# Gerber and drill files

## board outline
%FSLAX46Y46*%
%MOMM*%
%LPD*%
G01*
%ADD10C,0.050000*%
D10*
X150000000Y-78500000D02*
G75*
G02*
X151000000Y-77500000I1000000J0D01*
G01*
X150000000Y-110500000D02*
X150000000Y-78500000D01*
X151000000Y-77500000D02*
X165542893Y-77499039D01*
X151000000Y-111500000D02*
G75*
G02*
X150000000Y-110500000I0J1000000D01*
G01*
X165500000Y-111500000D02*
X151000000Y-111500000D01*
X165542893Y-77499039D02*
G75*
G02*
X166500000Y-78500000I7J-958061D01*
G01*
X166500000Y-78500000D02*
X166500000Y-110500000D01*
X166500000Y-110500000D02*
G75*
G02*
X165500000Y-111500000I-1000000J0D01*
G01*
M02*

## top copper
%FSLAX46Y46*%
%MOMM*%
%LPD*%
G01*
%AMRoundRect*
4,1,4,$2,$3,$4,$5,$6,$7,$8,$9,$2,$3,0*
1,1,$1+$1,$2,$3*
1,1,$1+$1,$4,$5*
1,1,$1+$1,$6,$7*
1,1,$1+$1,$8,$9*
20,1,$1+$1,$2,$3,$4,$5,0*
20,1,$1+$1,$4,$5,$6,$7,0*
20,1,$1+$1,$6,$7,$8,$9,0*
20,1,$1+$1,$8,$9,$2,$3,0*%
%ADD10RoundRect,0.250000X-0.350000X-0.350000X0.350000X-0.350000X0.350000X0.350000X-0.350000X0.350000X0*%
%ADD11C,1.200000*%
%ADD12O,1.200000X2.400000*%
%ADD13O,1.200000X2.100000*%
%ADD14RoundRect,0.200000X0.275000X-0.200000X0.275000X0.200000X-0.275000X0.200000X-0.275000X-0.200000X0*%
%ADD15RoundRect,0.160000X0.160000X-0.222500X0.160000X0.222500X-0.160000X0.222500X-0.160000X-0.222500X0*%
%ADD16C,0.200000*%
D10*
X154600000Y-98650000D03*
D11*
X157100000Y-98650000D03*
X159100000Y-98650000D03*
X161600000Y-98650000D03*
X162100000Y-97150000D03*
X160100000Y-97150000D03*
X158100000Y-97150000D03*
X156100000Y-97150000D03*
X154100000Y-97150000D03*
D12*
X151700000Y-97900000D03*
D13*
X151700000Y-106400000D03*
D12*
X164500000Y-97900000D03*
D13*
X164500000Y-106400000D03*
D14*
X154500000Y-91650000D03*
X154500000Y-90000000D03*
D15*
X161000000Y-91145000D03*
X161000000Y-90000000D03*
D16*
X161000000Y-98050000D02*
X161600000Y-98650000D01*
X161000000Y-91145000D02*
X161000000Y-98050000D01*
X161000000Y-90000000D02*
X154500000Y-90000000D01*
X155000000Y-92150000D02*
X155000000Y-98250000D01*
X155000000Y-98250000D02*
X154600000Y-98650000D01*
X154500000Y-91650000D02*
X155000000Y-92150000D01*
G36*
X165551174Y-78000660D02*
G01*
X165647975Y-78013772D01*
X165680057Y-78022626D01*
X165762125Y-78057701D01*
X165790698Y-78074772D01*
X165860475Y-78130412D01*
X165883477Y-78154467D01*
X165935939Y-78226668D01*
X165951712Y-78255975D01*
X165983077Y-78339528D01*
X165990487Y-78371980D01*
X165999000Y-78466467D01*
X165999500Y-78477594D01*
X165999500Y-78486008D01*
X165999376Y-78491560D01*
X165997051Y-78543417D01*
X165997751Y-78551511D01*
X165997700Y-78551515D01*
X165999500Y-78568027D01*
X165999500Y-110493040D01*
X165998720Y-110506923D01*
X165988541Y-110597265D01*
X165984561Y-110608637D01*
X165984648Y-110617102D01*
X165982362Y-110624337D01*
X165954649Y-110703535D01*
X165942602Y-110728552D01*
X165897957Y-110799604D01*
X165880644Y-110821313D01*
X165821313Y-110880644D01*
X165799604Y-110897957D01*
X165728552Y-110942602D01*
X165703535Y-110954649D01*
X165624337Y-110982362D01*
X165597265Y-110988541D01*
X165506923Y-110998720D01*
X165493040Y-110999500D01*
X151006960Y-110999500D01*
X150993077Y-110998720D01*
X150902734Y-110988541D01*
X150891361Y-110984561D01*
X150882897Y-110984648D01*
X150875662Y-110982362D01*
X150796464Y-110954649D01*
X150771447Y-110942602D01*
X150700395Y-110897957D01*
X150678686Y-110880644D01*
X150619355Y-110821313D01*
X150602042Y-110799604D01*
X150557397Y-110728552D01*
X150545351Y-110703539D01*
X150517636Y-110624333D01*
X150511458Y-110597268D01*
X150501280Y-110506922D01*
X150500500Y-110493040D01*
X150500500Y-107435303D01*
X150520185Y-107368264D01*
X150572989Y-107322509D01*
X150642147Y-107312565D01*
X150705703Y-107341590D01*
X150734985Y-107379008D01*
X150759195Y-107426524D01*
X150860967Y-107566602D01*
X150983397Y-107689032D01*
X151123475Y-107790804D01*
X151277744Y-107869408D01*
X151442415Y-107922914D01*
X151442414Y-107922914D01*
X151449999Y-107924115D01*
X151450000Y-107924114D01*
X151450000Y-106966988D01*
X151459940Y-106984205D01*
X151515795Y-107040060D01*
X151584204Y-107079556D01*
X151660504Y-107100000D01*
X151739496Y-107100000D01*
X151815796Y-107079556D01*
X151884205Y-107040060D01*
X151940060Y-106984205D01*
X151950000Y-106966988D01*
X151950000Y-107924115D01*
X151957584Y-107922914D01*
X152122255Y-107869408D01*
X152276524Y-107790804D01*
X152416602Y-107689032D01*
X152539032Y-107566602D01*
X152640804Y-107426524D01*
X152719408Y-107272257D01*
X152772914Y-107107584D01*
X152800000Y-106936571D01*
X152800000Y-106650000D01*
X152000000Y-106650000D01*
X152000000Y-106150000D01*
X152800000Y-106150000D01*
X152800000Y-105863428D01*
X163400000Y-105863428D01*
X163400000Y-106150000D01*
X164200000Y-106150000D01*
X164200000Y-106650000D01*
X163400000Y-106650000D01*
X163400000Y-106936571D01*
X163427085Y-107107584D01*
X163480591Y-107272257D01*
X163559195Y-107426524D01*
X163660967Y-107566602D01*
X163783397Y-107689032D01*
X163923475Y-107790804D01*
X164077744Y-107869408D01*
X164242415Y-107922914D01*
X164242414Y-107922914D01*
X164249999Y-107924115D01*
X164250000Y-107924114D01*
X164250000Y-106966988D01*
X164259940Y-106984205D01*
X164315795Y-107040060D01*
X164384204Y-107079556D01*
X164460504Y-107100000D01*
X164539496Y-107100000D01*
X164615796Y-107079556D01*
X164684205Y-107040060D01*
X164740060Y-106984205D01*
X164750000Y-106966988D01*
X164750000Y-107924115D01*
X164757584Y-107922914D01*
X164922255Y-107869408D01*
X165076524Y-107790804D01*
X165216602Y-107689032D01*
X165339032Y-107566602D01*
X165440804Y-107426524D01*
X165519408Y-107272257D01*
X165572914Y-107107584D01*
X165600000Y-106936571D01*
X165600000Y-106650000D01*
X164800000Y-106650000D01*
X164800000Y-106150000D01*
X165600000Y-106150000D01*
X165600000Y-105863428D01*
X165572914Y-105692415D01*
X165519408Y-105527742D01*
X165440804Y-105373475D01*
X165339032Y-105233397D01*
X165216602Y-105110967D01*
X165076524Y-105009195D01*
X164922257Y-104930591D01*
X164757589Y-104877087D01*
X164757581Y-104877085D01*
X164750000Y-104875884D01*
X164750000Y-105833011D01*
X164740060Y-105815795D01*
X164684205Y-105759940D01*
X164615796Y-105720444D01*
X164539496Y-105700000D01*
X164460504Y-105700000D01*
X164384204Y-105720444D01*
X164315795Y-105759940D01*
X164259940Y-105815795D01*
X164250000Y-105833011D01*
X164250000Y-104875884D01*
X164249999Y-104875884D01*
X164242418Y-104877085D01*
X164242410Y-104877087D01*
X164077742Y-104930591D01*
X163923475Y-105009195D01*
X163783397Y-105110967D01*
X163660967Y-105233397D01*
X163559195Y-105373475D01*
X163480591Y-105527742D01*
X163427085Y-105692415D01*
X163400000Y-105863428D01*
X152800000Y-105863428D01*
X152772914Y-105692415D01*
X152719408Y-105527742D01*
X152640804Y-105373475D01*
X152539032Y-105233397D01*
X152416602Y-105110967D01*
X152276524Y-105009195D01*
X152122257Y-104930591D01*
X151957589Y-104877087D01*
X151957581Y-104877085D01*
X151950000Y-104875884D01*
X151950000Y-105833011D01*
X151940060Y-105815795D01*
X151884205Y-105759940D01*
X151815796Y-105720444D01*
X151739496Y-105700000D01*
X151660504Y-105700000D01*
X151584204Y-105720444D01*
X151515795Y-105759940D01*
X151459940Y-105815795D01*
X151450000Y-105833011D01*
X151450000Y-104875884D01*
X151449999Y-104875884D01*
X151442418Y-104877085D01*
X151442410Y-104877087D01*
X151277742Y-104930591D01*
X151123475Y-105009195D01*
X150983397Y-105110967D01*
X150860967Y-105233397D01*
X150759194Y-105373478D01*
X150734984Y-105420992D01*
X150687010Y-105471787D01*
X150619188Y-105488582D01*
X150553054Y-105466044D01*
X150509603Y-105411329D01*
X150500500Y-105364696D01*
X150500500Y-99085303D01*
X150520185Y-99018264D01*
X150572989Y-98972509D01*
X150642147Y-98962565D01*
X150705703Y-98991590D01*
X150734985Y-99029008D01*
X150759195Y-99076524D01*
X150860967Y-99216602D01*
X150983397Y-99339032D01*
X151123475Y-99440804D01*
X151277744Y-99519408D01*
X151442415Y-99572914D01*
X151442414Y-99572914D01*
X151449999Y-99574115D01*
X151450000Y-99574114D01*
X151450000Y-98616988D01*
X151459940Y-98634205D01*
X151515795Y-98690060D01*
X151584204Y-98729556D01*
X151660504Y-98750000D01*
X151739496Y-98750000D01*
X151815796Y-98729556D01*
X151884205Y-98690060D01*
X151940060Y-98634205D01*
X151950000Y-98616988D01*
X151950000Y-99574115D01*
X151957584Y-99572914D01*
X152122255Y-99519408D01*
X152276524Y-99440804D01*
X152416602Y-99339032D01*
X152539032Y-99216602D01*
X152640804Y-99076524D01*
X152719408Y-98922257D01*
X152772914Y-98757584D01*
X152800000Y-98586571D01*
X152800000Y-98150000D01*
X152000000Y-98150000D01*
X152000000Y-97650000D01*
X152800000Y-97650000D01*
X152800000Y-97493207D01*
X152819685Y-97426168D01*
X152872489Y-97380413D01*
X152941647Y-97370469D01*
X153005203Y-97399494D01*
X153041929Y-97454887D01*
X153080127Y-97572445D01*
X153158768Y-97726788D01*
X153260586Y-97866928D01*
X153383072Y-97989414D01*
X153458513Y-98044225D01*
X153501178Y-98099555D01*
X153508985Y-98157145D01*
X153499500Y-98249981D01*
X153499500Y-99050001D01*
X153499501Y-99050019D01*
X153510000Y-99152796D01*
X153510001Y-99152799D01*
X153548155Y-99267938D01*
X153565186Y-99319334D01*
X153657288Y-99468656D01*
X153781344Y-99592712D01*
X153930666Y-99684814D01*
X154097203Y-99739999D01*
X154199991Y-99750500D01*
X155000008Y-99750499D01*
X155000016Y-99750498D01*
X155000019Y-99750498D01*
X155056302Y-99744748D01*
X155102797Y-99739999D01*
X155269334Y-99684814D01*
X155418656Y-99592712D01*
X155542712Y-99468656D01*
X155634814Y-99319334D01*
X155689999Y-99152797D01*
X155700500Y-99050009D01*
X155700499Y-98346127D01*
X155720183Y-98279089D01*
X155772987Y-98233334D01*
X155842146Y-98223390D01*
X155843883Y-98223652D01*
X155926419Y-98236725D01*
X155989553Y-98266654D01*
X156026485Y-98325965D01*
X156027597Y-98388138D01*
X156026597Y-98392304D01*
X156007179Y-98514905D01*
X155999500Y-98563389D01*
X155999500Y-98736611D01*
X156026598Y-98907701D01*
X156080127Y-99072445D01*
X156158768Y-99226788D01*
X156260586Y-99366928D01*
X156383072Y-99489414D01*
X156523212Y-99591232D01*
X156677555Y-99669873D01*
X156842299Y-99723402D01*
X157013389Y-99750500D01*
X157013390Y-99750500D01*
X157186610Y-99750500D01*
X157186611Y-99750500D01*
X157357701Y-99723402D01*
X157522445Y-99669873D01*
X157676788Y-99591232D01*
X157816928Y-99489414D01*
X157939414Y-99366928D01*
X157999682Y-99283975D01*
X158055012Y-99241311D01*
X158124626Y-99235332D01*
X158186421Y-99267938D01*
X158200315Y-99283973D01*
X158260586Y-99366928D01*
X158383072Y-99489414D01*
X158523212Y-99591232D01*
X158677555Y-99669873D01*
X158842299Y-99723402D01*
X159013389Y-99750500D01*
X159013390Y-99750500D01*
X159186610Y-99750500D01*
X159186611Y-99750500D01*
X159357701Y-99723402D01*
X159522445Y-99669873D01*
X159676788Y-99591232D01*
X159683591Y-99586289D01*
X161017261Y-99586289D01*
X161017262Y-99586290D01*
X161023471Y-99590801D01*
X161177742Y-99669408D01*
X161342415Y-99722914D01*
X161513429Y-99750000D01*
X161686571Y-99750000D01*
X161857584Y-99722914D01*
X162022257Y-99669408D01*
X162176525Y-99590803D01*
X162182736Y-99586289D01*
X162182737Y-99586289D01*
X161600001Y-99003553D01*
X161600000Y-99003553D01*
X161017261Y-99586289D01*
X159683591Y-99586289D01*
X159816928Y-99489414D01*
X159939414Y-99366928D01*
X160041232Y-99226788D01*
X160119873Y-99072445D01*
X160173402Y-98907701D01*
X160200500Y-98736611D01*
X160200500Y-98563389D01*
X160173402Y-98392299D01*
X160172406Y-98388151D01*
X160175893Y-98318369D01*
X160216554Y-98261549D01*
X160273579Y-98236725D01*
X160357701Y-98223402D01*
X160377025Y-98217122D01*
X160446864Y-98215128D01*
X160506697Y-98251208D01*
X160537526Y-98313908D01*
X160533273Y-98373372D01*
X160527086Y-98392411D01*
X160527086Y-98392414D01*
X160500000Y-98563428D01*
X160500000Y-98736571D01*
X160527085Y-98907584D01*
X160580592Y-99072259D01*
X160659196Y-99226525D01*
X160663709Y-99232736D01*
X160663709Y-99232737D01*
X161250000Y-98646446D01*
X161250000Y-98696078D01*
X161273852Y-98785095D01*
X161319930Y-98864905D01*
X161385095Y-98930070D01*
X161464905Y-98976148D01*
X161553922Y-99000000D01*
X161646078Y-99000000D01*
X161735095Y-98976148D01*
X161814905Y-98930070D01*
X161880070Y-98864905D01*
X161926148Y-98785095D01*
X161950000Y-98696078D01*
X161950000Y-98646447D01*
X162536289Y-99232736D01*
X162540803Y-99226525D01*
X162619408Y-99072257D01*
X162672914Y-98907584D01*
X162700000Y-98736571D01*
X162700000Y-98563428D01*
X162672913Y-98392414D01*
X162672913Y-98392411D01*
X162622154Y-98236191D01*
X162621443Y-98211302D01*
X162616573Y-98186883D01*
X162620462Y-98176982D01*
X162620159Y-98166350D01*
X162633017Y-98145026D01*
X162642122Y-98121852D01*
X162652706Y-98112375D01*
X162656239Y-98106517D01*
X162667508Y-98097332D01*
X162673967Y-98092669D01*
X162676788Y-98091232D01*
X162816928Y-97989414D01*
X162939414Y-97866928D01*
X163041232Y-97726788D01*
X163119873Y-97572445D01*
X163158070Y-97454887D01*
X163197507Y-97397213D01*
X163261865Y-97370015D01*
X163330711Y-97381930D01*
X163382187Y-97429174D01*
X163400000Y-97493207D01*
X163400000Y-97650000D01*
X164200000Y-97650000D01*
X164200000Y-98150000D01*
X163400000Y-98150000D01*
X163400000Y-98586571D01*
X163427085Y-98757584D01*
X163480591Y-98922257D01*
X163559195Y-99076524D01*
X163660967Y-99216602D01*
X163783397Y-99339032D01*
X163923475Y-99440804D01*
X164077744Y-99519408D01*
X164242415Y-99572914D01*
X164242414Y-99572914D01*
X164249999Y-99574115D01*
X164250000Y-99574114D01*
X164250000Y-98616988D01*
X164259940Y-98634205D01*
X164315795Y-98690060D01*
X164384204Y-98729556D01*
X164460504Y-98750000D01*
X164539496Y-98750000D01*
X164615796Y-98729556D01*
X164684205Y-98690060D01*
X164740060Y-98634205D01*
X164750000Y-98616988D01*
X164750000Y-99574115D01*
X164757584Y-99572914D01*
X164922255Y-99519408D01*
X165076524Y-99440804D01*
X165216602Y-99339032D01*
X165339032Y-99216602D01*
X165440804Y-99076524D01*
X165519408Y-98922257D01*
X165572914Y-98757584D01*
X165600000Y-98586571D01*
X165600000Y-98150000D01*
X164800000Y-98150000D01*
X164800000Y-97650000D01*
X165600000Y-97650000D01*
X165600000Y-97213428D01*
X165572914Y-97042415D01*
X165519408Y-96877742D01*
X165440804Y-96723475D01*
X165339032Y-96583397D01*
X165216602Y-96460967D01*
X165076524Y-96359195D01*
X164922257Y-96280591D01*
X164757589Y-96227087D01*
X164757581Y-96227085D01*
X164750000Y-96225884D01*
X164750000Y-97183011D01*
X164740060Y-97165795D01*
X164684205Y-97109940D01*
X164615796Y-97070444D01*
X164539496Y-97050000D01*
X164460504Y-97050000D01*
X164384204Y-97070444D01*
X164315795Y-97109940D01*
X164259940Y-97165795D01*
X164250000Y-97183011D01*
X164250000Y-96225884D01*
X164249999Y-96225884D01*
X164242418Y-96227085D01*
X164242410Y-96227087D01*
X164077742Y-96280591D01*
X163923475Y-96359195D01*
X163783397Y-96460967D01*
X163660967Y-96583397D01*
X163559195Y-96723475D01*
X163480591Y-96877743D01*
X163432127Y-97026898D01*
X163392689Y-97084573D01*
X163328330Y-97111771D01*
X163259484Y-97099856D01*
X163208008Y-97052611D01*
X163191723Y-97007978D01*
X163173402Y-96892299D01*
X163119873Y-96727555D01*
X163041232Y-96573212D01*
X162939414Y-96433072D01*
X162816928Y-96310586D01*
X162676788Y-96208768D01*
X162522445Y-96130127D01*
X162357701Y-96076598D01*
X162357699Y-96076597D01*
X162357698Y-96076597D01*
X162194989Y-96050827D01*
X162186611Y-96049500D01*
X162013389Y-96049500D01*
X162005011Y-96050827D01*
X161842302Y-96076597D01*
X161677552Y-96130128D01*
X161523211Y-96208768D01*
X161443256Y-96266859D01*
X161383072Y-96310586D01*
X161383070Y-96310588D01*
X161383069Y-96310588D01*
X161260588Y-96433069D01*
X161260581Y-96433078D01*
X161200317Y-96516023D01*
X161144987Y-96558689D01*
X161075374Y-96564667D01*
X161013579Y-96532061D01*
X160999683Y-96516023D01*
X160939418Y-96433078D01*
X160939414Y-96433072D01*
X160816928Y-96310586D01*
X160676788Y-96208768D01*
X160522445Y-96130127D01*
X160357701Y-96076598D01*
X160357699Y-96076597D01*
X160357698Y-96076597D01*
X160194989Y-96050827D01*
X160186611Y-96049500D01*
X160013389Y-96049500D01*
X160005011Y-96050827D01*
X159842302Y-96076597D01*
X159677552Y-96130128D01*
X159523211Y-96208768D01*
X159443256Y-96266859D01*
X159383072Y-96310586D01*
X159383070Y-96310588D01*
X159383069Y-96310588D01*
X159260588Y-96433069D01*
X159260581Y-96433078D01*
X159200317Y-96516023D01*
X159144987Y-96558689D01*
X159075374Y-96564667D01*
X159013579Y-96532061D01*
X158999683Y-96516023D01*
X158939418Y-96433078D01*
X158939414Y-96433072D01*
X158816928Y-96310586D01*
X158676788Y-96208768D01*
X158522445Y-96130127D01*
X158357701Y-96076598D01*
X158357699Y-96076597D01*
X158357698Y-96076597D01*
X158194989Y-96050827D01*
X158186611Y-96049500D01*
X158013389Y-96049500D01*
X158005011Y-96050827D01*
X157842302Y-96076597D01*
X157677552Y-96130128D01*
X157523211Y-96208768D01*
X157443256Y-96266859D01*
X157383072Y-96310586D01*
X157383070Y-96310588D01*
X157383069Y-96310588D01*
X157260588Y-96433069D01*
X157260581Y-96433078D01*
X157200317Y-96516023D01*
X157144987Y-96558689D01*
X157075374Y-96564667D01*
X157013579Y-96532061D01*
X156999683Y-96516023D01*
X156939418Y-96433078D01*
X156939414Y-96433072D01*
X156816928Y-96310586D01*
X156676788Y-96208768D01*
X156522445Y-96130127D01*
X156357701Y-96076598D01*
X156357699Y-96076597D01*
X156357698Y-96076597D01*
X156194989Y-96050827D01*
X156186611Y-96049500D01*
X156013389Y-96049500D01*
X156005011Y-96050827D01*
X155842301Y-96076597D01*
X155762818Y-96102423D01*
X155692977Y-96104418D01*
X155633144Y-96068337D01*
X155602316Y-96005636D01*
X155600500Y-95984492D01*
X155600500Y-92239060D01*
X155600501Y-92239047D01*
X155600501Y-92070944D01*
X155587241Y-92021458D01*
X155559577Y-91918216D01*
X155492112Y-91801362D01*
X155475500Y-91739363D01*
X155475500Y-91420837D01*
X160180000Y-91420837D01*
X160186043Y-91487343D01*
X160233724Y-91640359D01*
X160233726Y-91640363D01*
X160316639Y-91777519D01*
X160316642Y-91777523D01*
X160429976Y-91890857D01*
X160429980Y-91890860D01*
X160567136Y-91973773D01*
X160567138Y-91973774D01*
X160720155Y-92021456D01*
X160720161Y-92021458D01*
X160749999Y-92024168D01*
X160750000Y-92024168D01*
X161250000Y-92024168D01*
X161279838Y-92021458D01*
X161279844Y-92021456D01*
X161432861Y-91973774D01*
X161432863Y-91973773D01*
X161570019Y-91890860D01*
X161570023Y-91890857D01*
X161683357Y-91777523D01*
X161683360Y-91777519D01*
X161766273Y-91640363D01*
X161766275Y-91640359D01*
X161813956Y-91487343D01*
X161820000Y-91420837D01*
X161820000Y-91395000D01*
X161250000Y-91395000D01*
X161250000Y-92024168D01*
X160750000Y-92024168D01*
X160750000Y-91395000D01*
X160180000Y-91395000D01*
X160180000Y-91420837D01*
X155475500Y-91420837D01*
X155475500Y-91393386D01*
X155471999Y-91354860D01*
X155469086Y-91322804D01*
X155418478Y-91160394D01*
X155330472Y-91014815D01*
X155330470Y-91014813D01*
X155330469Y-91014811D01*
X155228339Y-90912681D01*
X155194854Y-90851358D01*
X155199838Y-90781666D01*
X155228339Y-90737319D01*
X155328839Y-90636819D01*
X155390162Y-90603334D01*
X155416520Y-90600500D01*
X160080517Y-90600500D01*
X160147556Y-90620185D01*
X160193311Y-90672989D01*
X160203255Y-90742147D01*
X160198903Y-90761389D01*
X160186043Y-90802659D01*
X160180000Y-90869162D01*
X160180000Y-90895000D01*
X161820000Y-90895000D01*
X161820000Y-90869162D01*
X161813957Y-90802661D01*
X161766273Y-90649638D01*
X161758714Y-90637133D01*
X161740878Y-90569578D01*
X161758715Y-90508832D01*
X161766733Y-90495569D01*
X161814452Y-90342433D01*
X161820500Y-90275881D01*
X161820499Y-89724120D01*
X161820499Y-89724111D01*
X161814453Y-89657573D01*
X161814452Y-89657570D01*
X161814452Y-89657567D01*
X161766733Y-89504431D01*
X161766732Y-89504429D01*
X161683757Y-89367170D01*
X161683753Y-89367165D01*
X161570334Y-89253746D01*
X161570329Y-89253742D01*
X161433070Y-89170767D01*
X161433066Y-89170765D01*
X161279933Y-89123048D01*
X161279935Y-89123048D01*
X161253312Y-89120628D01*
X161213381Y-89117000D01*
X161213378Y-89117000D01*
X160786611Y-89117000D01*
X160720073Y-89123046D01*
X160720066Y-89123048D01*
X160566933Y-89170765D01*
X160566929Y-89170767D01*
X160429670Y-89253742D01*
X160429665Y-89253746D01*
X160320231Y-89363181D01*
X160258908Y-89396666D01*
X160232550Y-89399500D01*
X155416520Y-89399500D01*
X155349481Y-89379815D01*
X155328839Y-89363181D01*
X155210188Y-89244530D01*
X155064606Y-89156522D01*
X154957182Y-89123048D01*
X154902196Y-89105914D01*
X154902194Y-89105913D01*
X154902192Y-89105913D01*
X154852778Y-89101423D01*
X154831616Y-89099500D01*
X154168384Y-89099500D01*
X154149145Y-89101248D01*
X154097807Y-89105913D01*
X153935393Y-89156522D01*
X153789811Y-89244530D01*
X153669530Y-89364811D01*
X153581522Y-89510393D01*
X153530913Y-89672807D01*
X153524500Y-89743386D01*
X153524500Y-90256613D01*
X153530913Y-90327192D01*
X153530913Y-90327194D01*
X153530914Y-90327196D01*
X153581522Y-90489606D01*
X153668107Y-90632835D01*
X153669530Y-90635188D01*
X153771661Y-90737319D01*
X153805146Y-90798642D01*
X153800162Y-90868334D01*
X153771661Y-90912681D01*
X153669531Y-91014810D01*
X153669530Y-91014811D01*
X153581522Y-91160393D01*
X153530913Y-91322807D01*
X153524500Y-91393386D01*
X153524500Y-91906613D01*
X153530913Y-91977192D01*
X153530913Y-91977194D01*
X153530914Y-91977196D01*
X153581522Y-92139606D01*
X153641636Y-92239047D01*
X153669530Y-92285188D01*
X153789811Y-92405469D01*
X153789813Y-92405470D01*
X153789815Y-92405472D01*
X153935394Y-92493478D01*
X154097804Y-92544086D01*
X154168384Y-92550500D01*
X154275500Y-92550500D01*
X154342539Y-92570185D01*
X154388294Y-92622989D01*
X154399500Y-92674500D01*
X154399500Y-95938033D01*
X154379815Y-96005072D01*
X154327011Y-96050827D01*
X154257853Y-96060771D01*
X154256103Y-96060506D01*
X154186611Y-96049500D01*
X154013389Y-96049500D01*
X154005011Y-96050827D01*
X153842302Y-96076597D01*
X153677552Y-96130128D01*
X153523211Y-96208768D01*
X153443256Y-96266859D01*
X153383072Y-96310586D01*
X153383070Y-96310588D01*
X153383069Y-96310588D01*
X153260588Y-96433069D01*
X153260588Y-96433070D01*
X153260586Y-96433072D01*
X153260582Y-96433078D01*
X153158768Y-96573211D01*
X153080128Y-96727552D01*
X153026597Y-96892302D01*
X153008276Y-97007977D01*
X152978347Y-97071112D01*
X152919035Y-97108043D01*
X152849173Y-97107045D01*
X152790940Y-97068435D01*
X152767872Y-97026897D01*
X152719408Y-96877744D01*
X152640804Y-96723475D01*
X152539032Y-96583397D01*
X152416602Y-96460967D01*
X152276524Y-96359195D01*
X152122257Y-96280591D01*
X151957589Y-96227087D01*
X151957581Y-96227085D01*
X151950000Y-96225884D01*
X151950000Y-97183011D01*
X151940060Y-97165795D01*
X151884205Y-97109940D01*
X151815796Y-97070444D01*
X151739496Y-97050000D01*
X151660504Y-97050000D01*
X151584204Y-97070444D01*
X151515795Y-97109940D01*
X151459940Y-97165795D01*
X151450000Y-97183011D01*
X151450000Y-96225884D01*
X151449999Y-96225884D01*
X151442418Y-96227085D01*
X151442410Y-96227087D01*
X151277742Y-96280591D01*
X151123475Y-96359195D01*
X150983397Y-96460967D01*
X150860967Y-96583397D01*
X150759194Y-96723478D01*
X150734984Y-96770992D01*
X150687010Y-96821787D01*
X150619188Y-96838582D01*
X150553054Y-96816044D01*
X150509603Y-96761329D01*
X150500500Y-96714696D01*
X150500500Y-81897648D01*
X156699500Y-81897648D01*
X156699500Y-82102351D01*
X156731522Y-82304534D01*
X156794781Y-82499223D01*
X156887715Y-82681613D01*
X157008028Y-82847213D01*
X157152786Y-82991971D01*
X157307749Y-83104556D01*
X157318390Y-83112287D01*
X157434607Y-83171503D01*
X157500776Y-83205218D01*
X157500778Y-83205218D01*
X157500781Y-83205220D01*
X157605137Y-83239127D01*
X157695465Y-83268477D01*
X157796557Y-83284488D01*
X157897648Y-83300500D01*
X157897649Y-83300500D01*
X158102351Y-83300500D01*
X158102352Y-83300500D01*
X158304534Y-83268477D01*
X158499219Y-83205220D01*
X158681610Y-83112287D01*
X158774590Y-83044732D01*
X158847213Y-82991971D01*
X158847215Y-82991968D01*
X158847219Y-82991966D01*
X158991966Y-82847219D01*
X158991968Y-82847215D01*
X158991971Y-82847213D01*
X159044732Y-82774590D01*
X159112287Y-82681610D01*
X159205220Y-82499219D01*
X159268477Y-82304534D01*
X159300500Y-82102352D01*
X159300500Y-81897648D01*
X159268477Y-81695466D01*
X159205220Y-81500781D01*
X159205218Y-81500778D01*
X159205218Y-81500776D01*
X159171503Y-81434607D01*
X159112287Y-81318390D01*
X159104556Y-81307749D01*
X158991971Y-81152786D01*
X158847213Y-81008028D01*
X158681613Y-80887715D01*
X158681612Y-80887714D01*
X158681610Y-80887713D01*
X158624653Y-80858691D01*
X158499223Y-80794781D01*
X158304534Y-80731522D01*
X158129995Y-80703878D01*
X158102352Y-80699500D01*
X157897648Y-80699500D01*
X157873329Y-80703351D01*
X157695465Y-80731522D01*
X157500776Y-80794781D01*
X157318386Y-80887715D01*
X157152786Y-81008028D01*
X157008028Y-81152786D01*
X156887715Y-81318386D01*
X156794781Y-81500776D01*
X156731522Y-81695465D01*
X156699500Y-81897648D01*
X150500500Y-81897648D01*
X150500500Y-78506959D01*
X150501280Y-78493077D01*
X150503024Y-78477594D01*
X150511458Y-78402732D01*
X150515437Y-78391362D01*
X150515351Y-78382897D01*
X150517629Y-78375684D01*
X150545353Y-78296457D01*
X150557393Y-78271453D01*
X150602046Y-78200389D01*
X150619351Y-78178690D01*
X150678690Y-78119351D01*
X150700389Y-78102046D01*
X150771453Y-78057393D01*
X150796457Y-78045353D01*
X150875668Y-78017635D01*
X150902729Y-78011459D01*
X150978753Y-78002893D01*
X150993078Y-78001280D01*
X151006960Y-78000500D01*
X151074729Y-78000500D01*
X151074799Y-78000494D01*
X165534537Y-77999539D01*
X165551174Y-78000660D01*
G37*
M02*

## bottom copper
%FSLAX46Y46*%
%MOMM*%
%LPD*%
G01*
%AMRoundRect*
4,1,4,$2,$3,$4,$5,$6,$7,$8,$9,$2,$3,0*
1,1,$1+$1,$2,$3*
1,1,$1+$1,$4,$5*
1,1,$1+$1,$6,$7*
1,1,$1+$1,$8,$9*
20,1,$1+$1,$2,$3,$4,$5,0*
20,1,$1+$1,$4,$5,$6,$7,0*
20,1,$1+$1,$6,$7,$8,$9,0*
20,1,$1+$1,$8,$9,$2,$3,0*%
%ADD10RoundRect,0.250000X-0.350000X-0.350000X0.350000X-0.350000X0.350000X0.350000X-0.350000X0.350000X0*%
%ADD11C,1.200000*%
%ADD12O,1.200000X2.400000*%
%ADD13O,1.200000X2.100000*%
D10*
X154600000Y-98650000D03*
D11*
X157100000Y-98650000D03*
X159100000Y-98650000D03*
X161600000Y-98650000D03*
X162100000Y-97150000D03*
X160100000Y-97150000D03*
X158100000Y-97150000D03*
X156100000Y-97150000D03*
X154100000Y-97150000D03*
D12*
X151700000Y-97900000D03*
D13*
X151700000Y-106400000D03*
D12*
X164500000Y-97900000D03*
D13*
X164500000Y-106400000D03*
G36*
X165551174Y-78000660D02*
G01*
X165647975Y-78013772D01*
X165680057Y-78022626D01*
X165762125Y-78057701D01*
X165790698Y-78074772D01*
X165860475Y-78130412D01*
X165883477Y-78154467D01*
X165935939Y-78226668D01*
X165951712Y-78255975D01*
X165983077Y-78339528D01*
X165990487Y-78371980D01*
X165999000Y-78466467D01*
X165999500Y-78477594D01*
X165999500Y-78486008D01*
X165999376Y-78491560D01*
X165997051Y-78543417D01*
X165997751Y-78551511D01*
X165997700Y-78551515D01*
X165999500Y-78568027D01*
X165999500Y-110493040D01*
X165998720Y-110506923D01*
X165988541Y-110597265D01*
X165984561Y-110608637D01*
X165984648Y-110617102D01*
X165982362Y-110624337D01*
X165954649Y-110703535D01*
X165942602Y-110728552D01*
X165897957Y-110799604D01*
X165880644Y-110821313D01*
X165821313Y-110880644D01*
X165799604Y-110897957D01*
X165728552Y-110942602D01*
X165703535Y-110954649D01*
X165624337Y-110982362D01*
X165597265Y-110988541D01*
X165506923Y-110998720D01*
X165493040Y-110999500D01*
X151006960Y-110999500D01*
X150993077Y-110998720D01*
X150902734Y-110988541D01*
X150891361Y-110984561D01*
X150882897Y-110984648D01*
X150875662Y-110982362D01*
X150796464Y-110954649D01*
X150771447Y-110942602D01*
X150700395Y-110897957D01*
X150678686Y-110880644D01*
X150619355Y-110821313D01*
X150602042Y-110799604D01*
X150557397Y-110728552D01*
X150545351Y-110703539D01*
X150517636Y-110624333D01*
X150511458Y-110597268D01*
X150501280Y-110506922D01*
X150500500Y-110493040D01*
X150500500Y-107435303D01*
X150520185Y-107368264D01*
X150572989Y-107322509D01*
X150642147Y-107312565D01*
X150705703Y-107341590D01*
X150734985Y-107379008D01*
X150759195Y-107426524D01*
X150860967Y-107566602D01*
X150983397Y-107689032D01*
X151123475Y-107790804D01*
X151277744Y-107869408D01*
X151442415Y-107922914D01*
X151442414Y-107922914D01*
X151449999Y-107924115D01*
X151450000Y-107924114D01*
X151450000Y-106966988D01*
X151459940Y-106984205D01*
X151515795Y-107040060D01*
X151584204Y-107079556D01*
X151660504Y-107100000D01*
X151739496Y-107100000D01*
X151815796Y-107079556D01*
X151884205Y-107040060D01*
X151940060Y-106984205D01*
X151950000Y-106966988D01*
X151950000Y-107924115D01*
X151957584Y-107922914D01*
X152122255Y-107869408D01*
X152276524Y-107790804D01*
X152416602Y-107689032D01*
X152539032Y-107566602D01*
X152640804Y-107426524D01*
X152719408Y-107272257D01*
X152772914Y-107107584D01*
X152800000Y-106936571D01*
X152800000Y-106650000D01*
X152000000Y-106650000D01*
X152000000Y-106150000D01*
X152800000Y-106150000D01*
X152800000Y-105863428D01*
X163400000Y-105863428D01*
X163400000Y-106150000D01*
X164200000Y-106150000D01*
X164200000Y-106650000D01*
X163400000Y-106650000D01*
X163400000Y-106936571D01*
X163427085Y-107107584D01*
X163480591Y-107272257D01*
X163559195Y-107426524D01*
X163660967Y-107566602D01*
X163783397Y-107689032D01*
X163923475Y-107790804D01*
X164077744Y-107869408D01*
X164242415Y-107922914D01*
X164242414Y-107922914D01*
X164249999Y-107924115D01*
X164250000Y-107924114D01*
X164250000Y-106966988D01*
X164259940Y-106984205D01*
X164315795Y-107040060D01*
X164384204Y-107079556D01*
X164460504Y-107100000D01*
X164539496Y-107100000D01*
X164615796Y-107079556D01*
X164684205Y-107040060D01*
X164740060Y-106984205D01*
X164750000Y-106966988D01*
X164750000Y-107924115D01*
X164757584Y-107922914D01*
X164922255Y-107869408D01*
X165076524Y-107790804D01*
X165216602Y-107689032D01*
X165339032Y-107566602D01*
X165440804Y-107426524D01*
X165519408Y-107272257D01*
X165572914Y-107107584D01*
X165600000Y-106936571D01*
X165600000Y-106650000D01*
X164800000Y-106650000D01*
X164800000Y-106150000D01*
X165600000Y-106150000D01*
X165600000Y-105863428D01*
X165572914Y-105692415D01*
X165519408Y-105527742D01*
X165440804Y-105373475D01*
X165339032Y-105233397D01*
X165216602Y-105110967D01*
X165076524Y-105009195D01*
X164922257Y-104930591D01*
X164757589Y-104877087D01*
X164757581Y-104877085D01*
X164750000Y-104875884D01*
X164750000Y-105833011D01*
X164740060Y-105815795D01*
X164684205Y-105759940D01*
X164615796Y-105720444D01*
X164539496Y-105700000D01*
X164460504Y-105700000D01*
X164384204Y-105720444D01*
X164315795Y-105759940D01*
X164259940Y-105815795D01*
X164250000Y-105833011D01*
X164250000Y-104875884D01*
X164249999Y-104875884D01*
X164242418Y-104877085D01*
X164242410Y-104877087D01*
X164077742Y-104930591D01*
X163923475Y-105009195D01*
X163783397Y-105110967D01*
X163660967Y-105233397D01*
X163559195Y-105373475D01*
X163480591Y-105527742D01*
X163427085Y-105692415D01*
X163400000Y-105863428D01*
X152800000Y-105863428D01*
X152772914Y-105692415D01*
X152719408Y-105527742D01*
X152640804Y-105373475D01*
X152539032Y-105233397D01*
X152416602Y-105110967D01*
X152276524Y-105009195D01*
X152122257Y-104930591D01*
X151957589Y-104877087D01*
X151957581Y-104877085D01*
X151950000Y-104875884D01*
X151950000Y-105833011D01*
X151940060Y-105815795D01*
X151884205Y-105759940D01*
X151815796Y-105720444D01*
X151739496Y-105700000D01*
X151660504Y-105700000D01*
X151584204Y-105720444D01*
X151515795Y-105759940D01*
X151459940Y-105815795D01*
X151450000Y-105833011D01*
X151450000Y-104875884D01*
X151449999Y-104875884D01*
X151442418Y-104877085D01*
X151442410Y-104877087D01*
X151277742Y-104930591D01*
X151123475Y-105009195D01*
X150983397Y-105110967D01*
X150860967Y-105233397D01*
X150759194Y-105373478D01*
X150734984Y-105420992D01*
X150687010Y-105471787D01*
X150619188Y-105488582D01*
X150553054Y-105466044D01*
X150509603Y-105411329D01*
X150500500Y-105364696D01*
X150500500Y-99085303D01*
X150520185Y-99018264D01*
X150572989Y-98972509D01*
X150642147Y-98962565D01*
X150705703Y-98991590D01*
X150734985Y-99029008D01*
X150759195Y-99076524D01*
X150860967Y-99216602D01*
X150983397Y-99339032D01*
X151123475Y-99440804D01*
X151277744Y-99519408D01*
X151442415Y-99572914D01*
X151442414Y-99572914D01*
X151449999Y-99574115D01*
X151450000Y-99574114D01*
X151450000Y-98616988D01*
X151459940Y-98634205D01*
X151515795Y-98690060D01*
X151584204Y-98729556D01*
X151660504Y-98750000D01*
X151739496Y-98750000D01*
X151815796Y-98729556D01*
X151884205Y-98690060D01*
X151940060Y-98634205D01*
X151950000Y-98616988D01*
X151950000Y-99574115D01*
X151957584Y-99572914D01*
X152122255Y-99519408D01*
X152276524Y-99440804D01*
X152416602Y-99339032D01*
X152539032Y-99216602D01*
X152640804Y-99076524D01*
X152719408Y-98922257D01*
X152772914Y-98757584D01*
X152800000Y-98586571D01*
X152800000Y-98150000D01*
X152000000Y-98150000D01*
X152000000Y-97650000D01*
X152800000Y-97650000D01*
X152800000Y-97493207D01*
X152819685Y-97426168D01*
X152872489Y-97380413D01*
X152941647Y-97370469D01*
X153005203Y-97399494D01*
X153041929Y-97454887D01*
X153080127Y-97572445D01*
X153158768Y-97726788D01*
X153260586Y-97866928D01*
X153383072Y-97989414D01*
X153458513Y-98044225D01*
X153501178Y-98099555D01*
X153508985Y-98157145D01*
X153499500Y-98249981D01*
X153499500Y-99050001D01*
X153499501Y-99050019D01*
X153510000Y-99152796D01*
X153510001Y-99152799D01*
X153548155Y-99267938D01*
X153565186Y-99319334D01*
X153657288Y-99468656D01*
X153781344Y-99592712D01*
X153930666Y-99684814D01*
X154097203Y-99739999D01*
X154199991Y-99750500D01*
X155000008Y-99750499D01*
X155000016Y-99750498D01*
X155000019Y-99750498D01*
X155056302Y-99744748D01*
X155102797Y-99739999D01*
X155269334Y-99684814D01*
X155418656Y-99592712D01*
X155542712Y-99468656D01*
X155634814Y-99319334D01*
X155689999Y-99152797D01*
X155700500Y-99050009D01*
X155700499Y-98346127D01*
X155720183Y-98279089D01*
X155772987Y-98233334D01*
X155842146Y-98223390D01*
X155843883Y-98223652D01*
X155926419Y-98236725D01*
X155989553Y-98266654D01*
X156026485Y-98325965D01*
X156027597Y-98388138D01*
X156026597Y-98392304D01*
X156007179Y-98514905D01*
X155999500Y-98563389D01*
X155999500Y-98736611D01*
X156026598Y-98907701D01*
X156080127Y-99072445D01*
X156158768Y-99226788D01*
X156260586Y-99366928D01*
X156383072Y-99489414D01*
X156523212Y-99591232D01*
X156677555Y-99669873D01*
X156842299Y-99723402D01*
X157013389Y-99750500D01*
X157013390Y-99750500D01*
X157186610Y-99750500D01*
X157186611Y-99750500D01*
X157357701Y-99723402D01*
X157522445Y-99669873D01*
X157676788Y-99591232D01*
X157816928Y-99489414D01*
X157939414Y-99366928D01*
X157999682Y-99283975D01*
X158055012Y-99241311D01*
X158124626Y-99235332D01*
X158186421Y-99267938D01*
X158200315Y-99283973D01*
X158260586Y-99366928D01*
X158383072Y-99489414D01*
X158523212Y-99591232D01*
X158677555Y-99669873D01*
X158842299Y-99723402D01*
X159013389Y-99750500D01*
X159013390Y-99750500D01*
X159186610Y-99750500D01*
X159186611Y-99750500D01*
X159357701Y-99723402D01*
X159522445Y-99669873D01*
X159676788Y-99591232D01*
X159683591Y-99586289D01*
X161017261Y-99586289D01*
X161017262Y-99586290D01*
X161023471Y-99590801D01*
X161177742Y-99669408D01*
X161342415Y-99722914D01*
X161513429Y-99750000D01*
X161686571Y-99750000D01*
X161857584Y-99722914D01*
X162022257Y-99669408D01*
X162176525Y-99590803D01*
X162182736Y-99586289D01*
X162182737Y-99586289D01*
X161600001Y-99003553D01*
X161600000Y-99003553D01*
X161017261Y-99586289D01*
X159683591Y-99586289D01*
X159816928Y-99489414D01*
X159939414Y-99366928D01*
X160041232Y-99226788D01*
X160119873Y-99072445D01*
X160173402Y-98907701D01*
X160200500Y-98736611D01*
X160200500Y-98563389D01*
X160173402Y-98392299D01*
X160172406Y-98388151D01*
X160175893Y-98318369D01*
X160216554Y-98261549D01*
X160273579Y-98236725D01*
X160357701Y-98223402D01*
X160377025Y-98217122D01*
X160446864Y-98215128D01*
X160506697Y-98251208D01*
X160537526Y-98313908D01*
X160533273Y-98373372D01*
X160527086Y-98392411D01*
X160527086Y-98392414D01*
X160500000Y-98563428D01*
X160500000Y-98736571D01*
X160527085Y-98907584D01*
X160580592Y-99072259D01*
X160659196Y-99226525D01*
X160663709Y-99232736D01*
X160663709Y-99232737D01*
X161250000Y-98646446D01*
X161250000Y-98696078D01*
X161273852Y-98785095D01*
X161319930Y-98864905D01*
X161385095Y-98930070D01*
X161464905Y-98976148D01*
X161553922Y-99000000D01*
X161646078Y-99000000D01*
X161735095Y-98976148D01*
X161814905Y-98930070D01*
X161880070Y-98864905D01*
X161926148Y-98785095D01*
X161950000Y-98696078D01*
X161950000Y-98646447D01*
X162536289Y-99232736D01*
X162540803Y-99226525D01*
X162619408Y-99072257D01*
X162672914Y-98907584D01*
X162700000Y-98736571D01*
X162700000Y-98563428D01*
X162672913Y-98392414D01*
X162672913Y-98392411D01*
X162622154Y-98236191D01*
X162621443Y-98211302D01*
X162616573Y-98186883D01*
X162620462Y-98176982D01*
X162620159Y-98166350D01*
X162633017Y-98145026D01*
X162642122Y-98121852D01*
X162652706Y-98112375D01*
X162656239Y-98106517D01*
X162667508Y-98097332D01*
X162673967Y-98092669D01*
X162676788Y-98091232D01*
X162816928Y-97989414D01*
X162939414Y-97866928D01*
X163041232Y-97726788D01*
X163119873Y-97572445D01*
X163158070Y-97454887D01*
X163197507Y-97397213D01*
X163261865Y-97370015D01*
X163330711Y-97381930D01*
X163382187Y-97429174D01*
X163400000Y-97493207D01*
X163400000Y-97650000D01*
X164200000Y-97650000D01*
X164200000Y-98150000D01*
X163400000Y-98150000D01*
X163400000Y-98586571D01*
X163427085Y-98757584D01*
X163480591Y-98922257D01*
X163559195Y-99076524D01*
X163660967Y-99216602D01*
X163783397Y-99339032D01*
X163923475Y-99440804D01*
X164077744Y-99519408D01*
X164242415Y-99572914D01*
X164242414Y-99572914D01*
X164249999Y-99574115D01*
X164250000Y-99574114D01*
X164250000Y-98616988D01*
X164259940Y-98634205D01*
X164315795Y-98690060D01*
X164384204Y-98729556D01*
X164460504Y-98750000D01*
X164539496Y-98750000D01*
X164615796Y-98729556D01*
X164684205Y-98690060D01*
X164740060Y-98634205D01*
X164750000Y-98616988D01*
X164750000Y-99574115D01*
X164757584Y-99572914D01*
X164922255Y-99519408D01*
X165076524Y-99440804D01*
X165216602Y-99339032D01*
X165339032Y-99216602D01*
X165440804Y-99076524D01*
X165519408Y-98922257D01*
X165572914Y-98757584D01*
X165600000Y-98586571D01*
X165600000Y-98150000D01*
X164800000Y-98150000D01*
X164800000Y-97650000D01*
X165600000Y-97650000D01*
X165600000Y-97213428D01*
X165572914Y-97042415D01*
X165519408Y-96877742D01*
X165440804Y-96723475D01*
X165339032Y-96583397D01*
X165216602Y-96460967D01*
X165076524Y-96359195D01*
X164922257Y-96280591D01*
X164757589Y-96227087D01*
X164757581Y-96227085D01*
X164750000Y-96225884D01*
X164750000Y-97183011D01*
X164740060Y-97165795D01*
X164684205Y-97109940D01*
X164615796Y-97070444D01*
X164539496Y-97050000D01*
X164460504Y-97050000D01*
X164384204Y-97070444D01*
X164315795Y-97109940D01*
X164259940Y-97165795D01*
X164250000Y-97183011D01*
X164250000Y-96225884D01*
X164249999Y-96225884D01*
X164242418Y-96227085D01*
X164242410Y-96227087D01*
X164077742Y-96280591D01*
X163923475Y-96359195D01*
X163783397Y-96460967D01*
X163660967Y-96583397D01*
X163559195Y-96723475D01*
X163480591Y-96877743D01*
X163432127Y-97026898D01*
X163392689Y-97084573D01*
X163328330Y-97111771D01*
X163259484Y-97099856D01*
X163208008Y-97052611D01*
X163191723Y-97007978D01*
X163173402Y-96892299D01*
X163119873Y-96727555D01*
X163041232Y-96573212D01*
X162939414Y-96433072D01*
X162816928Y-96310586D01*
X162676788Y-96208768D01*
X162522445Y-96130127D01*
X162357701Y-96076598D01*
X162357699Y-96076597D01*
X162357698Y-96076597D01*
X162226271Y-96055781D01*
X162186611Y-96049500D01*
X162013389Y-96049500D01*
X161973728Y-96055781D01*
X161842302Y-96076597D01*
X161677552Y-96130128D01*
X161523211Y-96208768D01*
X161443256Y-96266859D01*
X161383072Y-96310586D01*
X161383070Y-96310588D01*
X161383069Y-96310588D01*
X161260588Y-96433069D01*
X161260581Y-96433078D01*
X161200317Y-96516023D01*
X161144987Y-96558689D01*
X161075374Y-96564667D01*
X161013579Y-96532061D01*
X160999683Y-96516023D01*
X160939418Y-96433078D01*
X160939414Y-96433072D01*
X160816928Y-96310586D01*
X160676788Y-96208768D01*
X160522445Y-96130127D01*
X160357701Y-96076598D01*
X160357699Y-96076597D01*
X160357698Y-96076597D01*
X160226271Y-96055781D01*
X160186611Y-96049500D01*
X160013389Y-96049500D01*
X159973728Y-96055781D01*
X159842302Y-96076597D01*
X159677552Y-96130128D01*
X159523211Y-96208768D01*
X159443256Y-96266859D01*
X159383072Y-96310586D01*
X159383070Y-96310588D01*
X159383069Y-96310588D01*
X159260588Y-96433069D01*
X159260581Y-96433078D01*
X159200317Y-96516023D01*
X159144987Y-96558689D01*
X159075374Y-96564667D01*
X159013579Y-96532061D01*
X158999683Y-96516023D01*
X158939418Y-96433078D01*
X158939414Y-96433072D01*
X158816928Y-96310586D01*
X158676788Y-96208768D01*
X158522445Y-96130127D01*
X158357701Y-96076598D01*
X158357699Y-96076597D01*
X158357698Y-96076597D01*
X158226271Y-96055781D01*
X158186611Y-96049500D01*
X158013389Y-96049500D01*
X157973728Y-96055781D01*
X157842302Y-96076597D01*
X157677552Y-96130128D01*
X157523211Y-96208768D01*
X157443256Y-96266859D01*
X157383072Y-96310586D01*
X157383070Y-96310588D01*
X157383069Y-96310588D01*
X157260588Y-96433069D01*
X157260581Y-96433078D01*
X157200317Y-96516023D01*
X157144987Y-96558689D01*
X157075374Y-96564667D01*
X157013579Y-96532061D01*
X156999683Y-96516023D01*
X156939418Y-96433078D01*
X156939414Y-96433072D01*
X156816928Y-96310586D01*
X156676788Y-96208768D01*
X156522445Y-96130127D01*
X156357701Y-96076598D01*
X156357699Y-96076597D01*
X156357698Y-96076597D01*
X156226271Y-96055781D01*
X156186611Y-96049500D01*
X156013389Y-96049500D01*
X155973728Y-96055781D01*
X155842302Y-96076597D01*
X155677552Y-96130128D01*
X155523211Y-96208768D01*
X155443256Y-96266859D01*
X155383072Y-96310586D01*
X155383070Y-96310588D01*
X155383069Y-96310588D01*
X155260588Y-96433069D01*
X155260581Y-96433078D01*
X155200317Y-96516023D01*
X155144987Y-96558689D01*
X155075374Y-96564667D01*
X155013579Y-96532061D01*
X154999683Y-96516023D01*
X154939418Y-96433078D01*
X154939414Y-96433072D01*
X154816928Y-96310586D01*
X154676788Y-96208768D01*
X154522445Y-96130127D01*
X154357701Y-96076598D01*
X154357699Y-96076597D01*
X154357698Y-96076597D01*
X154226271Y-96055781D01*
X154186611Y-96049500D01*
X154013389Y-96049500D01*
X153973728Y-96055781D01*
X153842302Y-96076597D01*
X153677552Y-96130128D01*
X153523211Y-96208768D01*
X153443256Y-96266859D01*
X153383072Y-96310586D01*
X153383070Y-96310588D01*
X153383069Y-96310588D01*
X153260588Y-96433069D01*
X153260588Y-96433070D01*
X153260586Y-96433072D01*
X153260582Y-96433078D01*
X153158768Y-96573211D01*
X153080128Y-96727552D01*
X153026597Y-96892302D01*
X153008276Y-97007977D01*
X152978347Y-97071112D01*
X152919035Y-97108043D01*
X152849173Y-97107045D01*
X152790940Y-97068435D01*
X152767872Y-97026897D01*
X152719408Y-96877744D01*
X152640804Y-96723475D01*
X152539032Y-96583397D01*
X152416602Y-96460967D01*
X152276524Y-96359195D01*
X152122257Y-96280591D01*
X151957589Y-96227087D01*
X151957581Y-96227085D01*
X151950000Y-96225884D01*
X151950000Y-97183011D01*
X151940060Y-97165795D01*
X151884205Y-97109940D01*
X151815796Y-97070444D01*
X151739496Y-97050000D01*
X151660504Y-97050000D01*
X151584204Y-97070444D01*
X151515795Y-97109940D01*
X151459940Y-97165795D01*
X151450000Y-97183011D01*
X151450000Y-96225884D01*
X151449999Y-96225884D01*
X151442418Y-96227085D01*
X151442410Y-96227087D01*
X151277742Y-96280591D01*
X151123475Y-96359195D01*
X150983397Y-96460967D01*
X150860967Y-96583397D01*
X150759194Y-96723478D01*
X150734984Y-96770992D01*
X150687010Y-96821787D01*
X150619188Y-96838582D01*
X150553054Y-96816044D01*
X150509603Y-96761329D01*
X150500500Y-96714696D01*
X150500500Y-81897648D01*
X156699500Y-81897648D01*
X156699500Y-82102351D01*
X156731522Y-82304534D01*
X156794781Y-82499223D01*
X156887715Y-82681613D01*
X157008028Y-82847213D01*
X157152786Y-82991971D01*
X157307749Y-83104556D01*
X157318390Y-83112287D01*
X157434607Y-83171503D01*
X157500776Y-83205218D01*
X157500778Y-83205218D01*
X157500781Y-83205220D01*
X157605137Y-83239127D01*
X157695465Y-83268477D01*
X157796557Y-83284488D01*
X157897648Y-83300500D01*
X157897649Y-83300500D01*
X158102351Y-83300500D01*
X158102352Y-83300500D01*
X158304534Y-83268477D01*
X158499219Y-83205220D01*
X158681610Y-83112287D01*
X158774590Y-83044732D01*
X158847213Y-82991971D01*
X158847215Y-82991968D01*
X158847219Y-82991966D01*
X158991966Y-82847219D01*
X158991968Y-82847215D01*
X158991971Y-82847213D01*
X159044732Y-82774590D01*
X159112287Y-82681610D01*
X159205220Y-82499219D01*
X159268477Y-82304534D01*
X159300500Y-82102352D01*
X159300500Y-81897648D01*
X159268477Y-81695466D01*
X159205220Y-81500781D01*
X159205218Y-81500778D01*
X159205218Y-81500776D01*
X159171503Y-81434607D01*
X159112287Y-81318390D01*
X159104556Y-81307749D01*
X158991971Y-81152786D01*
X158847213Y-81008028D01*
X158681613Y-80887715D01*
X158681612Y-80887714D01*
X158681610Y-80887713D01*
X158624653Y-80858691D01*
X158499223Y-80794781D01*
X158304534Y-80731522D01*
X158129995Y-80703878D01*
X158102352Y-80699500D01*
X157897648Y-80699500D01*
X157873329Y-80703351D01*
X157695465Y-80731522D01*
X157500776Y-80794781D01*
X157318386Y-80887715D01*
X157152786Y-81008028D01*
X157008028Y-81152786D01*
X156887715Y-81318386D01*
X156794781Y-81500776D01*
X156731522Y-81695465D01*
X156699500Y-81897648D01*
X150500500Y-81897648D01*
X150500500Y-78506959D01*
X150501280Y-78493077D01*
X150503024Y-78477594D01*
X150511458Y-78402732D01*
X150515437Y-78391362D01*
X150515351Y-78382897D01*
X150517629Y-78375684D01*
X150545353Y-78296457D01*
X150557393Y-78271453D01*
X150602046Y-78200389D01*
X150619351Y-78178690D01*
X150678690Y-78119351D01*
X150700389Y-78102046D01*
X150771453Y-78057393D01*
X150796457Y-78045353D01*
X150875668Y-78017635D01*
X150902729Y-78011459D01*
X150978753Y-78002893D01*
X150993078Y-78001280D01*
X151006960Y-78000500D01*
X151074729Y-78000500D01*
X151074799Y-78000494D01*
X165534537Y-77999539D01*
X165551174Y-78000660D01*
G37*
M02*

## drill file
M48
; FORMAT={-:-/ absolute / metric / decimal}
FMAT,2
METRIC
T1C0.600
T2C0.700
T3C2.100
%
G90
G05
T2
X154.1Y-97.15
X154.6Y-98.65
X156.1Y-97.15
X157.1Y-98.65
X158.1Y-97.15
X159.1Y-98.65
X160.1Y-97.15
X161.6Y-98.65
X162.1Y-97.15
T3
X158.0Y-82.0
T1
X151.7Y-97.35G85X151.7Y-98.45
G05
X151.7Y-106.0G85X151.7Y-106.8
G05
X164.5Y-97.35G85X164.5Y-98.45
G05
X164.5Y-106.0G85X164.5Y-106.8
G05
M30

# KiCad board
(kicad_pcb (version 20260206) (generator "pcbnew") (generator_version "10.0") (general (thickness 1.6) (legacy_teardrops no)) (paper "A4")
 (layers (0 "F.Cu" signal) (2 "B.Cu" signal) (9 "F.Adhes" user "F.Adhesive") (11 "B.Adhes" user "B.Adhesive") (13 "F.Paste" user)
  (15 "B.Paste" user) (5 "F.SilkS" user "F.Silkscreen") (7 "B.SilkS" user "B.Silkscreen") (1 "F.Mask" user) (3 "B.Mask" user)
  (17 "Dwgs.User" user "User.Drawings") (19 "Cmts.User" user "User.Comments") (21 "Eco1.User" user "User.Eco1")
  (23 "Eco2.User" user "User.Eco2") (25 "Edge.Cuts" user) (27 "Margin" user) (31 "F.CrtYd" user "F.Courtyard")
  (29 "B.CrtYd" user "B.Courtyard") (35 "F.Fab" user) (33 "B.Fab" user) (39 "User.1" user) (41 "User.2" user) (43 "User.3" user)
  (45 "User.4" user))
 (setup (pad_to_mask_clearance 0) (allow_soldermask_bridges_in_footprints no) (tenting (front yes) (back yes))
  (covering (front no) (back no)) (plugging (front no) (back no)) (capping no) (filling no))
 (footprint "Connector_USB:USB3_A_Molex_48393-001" (layer "F.Cu") (at 154.6 98.65)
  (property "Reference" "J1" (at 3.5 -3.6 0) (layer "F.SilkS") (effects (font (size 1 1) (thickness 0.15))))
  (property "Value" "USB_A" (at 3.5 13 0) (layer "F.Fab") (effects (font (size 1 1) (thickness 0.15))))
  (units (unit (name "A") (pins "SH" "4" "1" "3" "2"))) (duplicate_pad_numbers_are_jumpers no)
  (pad "1" thru_hole roundrect (at 0 0) (size 1.2 1.2) (drill 0.7) (layers "*.Cu" "*.Mask") (remove_unused_layers no)
   (roundrect_rratio 0.2083333333) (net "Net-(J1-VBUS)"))
  (pad "2" thru_hole circle (at 2.5 0) (size 1.2 1.2) (drill 0.7) (layers "*.Cu" "*.Mask") (remove_unused_layers no)
   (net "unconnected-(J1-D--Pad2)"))
  (pad "3" thru_hole circle (at 4.5 0) (size 1.2 1.2) (drill 0.7) (layers "*.Cu" "*.Mask") (remove_unused_layers no)
   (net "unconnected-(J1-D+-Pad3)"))
  (pad "4" thru_hole circle (at 7 0) (size 1.2 1.2) (drill 0.7) (layers "*.Cu" "*.Mask") (remove_unused_layers no) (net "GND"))
  (pad "5" thru_hole circle (at 7.5 -1.5) (size 1.2 1.2) (drill 0.7) (layers "*.Cu" "*.Mask") (remove_unused_layers no))
  (pad "6" thru_hole circle (at 5.5 -1.5) (size 1.2 1.2) (drill 0.7) (layers "*.Cu" "*.Mask") (remove_unused_layers no))
  (pad "7" thru_hole circle (at 3.5 -1.5) (size 1.2 1.2) (drill 0.7) (layers "*.Cu" "*.Mask") (remove_unused_layers no))
  (pad "8" thru_hole circle (at 1.5 -1.5) (size 1.2 1.2) (drill 0.7) (layers "*.Cu" "*.Mask") (remove_unused_layers no))
  (pad "9" thru_hole circle (at -0.5 -1.5) (size 1.2 1.2) (drill 0.7) (layers "*.Cu" "*.Mask") (remove_unused_layers no))
  (pad "SH" thru_hole oval (at -2.9 -0.75) (size 1.2 2.4) (drill oval 0.6 1.7) (layers "*.Cu" "*.Mask") (remove_unused_layers no)
   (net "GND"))
  (pad "SH" thru_hole oval (at -2.9 7.75) (size 1.2 2.1) (drill oval 0.6 1.4) (layers "*.Cu" "*.Mask") (remove_unused_layers no) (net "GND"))
  (pad "SH" thru_hole oval (at 9.9 -0.75) (size 1.2 2.4) (drill oval 0.6 1.7) (layers "*.Cu" "*.Mask") (remove_unused_layers no) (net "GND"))
  (pad "SH" thru_hole oval (at 9.9 7.75) (size 1.2 2.1) (drill oval 0.6 1.4) (layers "*.Cu" "*.Mask") (remove_unused_layers no) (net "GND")))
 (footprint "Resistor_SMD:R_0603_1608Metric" (layer "F.Cu") (at 154.5 90.825 90)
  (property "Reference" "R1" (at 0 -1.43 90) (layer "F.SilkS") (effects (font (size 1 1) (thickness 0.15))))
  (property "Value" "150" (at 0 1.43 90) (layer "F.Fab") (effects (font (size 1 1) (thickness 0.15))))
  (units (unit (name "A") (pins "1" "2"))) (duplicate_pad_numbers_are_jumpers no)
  (pad "1" smd roundrect (at -0.825 0 90) (size 0.8 0.95) (layers "F.Cu" "F.Mask" "F.Paste") (roundrect_rratio 0.25) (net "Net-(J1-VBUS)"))
  (pad "2" smd roundrect (at 0.825 0 90) (size 0.8 0.95) (layers "F.Cu" "F.Mask" "F.Paste") (roundrect_rratio 0.25) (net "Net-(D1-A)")))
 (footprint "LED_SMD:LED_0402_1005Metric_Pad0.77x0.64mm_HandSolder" (layer "F.Cu") (at 161 90.5725 90)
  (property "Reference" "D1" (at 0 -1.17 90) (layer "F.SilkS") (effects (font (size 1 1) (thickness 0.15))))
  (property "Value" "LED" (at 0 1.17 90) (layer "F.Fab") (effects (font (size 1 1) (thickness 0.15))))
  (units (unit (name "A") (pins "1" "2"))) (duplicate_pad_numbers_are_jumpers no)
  (pad "1" smd roundrect (at -0.5725 0 90) (size 0.765 0.64) (layers "F.Cu" "F.Mask" "F.Paste") (roundrect_rratio 0.25) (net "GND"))
  (pad "2" smd roundrect (at 0.5725 0 90) (size 0.765 0.64) (layers "F.Cu" "F.Mask" "F.Paste") (roundrect_rratio 0.25) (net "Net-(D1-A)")))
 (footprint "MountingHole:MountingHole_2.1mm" (layer "F.Cu") (at 158 82)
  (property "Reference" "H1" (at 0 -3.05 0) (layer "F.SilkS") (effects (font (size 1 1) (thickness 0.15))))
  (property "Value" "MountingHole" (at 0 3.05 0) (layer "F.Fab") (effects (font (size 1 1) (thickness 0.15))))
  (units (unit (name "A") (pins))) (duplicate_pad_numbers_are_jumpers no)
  (pad "" np_thru_hole circle (at 0 0) (size 2.1 2.1) (drill 2.1) (layers "*.Cu" "*.Mask")))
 (gr_arc (start 150 78.5) (mid 150.292893 77.792893) (end 151 77.5) (stroke (width 0.05) (type default)) (layer "Edge.Cuts"))
 (gr_line (start 150 110.5) (end 150 78.5) (stroke (width 0.05) (type default)) (layer "Edge.Cuts"))
 (gr_line (start 151 77.5) (end 165.542893 77.499039) (stroke (width 0.05) (type default)) (layer "Edge.Cuts"))
 (gr_arc (start 151 111.5) (mid 150.292893 111.207107) (end 150 110.5) (stroke (width 0.05) (type default)) (layer "Edge.Cuts"))
 (gr_line (start 165.5 111.5) (end 151 111.5) (stroke (width 0.05) (type default)) (layer "Edge.Cuts"))
 (gr_arc (start 165.542893 77.499039) (mid 166.235348 77.794989) (end 166.5 78.5) (stroke (width 0.05) (type default)) (layer "Edge.Cuts"))
 (gr_line (start 166.5 78.5) (end 166.5 110.5) (stroke (width 0.05) (type default)) (layer "Edge.Cuts"))
 (gr_arc (start 166.5 110.5) (mid 166.207107 111.207107) (end 165.5 111.5) (stroke (width 0.05) (type default)) (layer "Edge.Cuts"))
 (segment (start 161 98.05) (end 161.6 98.65) (width 0.2) (layer "F.Cu") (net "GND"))
 (segment (start 161 91.145) (end 161 98.05) (width 0.2) (layer "F.Cu") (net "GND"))
 (segment (start 161 90) (end 154.5 90) (width 0.2) (layer "F.Cu") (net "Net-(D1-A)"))
 (segment (start 155 92.15) (end 155 98.25) (width 0.2) (layer "F.Cu") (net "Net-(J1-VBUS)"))
 (segment (start 155 98.25) (end 154.6 98.65) (width 0.2) (layer "F.Cu") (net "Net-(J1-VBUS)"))
 (segment (start 154.5 91.65) (end 155 92.15) (width 0.2) (layer "F.Cu") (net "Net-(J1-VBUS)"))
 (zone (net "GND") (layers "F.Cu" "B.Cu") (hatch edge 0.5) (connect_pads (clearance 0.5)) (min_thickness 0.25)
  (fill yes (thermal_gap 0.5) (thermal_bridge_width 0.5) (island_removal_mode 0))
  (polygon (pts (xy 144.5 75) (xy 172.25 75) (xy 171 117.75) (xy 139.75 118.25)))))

